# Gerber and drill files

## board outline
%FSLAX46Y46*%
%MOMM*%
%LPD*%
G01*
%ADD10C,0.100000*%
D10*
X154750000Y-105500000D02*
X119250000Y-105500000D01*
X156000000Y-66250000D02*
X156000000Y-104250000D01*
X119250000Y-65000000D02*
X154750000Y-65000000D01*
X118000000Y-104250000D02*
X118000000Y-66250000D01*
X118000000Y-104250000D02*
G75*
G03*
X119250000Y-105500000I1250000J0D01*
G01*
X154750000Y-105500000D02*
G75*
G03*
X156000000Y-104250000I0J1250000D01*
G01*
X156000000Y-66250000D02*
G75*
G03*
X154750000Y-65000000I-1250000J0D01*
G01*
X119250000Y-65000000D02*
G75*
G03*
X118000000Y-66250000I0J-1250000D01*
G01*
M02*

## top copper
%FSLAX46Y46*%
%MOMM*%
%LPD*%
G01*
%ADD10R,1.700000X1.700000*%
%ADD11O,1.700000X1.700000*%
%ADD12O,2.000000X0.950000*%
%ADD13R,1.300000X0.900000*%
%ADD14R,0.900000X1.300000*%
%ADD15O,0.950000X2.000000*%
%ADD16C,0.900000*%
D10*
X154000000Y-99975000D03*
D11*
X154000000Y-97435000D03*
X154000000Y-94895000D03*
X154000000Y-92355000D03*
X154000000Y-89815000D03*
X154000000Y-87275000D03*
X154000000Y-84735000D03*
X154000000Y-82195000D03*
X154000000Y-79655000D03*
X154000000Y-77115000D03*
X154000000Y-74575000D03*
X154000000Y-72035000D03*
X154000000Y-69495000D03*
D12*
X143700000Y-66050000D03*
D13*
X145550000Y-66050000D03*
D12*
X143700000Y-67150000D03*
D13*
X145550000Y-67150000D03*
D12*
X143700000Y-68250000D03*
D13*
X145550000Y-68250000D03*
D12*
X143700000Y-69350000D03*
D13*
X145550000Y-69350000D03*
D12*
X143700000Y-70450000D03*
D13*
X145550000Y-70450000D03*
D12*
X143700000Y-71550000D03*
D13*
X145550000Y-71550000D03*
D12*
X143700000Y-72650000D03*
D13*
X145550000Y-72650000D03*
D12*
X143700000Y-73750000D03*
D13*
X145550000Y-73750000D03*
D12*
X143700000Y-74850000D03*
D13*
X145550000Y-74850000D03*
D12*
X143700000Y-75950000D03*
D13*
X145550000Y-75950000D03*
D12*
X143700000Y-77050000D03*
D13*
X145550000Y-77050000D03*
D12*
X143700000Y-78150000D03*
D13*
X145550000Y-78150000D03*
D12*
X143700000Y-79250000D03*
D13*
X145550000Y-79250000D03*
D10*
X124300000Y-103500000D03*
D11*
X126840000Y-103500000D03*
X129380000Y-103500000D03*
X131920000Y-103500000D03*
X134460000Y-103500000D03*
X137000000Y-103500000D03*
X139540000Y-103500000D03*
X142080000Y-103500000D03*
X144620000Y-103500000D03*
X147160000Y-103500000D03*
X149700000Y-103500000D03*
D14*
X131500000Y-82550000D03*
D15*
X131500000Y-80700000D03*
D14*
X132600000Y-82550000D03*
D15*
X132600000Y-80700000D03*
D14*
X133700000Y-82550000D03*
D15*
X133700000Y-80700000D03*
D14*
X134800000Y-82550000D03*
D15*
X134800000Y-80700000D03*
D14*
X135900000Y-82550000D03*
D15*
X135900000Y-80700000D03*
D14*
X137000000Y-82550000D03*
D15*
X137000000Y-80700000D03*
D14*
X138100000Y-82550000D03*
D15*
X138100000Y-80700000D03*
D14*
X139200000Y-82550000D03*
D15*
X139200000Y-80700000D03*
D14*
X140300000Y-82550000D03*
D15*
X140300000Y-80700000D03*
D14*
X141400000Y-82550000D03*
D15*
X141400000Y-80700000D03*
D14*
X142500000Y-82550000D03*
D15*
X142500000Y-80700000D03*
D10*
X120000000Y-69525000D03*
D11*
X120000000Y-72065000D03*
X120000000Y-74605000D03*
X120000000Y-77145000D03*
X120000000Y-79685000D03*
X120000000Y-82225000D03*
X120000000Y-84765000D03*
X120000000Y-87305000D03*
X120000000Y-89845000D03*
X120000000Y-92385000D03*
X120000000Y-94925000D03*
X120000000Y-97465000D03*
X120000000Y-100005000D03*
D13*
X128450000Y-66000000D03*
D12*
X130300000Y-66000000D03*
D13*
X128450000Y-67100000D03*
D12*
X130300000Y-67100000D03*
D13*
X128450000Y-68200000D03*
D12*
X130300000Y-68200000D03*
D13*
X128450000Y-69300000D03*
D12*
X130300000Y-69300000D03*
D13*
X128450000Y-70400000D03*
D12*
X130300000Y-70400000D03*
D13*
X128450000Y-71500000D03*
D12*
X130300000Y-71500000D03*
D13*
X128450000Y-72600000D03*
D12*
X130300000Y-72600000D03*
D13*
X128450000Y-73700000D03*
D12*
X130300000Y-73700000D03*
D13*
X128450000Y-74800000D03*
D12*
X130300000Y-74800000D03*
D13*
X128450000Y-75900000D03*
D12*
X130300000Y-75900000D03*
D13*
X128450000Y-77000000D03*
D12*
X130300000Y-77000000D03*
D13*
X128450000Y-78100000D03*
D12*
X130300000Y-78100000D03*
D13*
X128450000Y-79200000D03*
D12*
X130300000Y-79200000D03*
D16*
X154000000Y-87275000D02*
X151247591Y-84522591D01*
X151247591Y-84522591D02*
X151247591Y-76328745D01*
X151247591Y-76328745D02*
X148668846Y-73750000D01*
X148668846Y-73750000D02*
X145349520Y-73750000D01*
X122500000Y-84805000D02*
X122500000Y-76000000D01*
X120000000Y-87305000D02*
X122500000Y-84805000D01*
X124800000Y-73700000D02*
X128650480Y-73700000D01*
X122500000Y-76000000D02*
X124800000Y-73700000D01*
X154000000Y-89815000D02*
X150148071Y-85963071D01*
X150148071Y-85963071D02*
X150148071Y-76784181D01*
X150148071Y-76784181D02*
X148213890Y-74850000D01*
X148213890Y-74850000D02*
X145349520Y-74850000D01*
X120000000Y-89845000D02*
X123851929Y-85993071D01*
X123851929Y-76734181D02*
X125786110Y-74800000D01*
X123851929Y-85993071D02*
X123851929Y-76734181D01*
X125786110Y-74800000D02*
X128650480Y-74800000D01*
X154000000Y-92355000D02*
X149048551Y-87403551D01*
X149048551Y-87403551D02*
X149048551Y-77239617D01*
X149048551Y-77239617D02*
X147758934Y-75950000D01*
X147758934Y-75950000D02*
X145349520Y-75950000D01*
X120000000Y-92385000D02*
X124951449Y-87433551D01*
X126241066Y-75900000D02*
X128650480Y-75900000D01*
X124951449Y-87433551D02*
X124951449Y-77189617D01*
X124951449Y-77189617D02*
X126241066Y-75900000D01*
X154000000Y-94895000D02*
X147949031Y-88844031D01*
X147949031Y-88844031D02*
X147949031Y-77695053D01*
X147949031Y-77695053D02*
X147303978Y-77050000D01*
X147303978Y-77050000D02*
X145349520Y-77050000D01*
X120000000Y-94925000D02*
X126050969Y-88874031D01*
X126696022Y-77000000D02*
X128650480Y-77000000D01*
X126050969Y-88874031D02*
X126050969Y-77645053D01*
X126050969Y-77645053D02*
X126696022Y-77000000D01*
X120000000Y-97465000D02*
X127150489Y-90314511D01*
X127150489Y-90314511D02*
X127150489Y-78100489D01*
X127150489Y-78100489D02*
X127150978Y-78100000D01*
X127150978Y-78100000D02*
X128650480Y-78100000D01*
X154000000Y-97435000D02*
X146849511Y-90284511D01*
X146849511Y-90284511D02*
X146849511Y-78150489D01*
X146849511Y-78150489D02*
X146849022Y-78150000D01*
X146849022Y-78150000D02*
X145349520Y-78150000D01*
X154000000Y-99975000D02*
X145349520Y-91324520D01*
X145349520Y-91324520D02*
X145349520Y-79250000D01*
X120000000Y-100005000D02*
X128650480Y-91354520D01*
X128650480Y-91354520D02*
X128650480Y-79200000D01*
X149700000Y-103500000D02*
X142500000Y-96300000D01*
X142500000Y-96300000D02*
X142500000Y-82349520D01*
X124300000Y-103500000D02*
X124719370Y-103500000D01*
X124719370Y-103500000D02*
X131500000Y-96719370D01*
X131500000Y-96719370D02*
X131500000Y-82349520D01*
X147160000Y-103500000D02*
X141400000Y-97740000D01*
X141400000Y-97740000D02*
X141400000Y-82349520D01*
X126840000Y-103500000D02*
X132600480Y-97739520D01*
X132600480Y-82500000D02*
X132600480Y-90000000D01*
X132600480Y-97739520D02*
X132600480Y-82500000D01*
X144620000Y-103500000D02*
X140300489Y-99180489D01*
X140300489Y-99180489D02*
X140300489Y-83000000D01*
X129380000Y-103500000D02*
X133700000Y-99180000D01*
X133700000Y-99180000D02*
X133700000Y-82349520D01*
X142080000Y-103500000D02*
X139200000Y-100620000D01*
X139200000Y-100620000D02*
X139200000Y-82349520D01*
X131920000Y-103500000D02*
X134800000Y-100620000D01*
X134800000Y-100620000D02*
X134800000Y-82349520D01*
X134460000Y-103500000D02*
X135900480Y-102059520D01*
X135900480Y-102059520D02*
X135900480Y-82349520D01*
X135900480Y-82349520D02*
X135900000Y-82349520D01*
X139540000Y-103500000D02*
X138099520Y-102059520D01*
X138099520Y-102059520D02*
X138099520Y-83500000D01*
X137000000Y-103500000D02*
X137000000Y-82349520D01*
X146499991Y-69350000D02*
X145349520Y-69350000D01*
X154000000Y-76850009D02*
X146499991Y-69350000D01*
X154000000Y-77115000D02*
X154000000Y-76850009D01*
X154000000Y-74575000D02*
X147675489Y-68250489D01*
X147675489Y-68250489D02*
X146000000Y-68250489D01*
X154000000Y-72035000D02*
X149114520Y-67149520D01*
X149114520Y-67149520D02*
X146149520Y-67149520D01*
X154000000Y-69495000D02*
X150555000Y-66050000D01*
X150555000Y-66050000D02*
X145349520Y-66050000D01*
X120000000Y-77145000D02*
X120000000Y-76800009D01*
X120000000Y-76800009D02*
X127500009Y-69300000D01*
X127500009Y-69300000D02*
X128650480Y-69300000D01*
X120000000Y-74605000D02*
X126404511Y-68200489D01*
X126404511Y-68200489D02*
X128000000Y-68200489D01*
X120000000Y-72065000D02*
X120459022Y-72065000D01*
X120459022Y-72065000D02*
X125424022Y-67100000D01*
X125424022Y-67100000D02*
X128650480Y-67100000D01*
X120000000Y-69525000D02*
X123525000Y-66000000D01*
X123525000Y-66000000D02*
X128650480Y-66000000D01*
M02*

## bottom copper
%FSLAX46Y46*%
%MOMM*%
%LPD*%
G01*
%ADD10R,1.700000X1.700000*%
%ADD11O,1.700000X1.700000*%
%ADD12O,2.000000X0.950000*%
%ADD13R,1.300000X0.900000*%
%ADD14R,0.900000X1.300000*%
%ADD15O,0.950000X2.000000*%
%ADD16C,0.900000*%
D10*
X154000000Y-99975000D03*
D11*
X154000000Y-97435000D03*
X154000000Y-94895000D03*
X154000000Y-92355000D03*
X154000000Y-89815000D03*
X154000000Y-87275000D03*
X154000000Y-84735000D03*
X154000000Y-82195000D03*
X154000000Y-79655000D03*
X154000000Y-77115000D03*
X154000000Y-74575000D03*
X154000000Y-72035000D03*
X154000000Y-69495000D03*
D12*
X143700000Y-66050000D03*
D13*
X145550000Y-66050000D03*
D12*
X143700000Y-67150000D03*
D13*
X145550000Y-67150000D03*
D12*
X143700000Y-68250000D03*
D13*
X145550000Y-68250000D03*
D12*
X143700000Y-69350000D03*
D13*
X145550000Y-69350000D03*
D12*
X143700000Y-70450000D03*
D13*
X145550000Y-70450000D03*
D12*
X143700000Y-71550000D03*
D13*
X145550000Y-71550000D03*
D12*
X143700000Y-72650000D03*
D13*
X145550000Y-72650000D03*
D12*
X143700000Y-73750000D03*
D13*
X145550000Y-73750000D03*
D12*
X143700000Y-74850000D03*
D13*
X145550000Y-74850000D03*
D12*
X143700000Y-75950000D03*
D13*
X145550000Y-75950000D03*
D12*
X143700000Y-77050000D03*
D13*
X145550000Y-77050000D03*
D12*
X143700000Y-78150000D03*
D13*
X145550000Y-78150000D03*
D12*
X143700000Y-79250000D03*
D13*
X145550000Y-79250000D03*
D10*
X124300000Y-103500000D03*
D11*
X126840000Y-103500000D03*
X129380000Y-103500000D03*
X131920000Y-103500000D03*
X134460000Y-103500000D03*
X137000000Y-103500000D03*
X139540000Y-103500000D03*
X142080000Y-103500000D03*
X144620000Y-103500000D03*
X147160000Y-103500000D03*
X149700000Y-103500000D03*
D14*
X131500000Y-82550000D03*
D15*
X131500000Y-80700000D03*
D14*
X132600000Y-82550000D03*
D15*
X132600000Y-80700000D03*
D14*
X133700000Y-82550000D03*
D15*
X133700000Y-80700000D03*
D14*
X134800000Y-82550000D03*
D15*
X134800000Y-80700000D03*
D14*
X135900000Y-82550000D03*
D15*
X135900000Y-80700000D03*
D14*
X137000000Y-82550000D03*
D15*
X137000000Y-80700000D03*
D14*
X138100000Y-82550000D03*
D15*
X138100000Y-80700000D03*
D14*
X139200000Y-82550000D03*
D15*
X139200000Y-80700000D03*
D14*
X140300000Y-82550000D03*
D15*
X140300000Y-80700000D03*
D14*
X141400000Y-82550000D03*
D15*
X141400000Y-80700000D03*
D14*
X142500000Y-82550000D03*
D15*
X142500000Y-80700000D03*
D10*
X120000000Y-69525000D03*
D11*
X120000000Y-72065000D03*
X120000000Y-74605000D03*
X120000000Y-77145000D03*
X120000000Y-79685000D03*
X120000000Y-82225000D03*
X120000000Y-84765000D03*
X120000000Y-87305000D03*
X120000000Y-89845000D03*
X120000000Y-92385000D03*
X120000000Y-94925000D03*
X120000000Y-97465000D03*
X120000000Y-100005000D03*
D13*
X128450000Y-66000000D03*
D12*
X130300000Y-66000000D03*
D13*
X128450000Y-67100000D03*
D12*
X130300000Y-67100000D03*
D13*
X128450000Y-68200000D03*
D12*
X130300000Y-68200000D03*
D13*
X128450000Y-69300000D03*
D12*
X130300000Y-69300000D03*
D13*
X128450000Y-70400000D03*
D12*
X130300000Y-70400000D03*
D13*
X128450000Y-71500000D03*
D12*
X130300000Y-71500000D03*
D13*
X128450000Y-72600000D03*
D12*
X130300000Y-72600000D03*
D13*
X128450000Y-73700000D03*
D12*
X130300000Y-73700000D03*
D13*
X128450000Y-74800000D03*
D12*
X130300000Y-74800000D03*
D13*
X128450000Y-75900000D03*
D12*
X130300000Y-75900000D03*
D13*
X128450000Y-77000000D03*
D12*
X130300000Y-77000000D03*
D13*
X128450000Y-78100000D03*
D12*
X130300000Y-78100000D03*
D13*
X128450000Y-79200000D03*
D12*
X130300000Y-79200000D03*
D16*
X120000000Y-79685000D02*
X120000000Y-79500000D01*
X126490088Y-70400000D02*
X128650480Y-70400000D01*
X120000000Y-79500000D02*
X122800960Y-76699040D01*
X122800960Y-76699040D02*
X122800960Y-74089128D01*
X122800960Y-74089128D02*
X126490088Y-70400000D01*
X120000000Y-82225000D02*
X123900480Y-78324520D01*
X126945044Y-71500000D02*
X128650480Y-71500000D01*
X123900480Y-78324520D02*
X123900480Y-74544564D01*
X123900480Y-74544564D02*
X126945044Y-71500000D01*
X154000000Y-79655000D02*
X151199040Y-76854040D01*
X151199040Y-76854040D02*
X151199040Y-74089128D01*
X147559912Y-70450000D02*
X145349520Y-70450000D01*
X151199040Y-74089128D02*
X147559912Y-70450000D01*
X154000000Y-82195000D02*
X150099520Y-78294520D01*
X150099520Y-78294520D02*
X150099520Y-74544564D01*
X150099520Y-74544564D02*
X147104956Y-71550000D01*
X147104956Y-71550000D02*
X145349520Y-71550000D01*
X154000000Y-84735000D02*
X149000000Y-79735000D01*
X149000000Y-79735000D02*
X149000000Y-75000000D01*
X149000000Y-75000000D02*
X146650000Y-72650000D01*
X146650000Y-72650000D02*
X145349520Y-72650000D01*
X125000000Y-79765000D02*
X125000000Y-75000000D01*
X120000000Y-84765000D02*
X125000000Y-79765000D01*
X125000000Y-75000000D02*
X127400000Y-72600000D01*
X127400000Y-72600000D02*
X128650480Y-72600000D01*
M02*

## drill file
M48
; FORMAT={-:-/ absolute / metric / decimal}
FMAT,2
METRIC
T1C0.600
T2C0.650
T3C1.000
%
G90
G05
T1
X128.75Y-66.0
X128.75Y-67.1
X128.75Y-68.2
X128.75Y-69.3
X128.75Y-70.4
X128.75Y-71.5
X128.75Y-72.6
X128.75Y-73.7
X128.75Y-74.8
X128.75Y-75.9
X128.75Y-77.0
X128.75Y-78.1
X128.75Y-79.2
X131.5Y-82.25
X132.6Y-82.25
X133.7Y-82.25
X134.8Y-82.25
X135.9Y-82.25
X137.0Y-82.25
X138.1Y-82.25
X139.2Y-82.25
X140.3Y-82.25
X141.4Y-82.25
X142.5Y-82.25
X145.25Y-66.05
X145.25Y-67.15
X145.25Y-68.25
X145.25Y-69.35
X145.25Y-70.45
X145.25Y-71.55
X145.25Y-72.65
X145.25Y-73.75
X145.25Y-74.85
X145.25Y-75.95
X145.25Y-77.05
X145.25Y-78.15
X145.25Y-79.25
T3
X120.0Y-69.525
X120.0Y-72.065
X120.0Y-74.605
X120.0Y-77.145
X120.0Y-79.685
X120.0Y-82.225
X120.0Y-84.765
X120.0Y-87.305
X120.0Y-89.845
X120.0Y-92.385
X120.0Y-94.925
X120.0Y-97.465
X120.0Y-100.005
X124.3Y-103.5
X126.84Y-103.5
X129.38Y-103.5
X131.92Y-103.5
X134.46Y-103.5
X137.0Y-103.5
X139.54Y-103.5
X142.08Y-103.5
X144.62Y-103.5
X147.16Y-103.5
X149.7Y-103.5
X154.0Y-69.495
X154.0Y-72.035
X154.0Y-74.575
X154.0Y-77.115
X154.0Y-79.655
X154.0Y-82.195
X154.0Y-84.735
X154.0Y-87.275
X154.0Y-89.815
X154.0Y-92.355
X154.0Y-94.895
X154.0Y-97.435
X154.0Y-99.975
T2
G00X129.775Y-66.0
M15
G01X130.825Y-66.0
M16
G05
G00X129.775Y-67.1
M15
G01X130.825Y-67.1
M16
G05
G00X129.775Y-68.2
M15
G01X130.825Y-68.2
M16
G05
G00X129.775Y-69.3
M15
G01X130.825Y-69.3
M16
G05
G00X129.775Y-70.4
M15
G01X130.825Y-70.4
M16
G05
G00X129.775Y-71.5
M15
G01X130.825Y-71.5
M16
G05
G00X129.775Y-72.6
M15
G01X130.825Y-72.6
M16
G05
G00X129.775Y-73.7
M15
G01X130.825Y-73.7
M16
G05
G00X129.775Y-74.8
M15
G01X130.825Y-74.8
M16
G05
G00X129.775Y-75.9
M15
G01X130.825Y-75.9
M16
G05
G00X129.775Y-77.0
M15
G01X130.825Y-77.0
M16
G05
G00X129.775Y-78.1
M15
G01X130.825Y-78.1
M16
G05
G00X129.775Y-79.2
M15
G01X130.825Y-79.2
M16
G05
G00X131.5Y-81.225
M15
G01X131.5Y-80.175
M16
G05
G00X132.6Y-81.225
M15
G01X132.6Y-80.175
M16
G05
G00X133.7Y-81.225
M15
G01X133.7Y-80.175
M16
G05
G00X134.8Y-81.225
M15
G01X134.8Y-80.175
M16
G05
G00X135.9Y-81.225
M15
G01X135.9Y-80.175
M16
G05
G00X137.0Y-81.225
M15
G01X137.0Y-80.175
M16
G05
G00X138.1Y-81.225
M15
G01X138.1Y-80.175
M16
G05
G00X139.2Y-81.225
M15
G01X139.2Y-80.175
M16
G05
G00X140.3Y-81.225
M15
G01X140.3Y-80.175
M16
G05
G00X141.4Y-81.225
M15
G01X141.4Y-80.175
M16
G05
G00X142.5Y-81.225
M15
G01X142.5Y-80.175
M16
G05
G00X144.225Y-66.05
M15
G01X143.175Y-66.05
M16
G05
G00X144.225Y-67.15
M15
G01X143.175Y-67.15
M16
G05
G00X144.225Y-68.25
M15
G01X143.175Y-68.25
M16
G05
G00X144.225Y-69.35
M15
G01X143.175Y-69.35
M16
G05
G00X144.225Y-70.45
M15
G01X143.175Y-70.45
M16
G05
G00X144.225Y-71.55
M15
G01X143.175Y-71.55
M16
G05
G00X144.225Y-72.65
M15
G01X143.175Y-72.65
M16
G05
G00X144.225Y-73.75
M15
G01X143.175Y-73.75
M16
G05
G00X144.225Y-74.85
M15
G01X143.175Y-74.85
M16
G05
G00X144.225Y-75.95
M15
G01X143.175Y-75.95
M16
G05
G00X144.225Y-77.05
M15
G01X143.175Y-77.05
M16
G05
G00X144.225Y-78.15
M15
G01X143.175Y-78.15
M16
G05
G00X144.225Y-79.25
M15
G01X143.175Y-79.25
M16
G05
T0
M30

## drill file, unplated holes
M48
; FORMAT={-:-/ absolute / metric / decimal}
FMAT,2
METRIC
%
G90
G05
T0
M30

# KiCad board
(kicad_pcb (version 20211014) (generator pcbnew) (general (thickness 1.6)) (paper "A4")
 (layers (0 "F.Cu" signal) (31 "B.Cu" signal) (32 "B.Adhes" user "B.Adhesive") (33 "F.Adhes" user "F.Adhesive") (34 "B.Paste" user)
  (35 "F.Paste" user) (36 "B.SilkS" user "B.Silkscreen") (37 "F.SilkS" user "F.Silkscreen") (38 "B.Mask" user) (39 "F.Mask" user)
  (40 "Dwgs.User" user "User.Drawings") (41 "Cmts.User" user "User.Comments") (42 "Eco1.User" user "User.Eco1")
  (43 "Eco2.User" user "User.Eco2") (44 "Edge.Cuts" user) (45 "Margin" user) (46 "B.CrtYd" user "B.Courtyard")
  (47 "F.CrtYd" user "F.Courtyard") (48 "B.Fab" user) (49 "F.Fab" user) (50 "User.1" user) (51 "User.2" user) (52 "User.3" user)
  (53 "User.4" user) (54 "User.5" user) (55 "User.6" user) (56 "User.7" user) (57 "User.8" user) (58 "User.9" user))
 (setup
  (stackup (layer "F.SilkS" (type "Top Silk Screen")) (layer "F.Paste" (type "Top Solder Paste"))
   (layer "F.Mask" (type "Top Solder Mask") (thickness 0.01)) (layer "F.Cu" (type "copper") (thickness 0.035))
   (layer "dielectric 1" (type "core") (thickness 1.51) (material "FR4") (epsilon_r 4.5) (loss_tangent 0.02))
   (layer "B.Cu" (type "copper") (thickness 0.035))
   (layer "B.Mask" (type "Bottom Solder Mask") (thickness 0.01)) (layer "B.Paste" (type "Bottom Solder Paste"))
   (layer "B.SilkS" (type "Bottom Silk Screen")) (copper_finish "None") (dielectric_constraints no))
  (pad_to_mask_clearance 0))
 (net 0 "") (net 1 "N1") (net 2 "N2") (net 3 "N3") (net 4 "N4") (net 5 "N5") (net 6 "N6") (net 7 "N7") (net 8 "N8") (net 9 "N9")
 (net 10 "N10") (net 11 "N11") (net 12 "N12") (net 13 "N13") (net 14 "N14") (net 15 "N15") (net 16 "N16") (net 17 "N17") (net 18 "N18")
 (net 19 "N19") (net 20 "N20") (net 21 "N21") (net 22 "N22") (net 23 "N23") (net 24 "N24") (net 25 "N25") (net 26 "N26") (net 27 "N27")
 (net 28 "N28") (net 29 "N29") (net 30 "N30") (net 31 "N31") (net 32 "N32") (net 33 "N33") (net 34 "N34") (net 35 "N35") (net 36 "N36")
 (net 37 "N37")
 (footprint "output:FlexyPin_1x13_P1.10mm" (layer "F.Cu") (at 128.75 66)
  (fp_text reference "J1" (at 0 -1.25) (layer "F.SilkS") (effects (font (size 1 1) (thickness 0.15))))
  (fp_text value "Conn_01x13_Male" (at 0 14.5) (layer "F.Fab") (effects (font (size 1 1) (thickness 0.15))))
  (pad "" thru_hole oval locked (at 1.55 12.1) (size 2 0.95) (drill oval 1.7 0.65) (layers *.Cu *.Mask))
  (pad "" thru_hole oval locked (at 1.55 5.5) (size 2 0.95) (drill oval 1.7 0.65) (layers *.Cu *.Mask))
  (pad "" thru_hole oval locked (at 1.55 13.2) (size 2 0.95) (drill oval 1.7 0.65) (layers *.Cu *.Mask))
  (pad "" thru_hole oval locked (at 1.55 8.8) (size 2 0.95) (drill oval 1.7 0.65) (layers *.Cu *.Mask))
  (pad "" thru_hole oval locked (at 1.55 4.4) (size 2 0.95) (drill oval 1.7 0.65) (layers *.Cu *.Mask))
  (pad "" thru_hole oval locked (at 1.55 9.9) (size 2 0.95) (drill oval 1.7 0.65) (layers *.Cu *.Mask))
  (pad "" thru_hole oval locked (at 1.55 3.3) (size 2 0.95) (drill oval 1.7 0.65) (layers *.Cu *.Mask))
  (pad "" thru_hole oval locked (at 1.55 0) (size 2 0.95) (drill oval 1.7 0.65) (layers *.Cu *.Mask))
  (pad "" thru_hole oval locked (at 1.55 2.2) (size 2 0.95) (drill oval 1.7 0.65) (layers *.Cu *.Mask))
  (pad "" thru_hole oval locked (at 1.55 1.1) (size 2 0.95) (drill oval 1.7 0.65) (layers *.Cu *.Mask))
  (pad "" thru_hole oval locked (at 1.55 11) (size 2 0.95) (drill oval 1.7 0.65) (layers *.Cu *.Mask))
  (pad "" thru_hole oval locked (at 1.55 6.6) (size 2 0.95) (drill oval 1.7 0.65) (layers *.Cu *.Mask))
  (pad "" thru_hole oval locked (at 1.55 7.7) (size 2 0.95) (drill oval 1.7 0.65) (layers *.Cu *.Mask))
  (pad "1" thru_hole rect locked (at 0 0) (size 1.3 0.9) (drill 0.6 (offset -0.3 0)) (layers *.Cu *.Mask) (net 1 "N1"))
  (pad "2" thru_hole rect locked (at 0 1.1) (size 1.3 0.9) (drill 0.6 (offset -0.3 0)) (layers *.Cu *.Mask) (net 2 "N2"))
  (pad "3" thru_hole rect locked (at 0 2.2) (size 1.3 0.9) (drill 0.6 (offset -0.3 0)) (layers *.Cu *.Mask) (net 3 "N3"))
  (pad "4" thru_hole rect locked (at 0 3.3) (size 1.3 0.9) (drill 0.6 (offset -0.3 0)) (layers *.Cu *.Mask) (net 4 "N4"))
  (pad "5" thru_hole rect locked (at 0 4.4) (size 1.3 0.9) (drill 0.6 (offset -0.3 0)) (layers *.Cu *.Mask) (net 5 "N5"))
  (pad "6" thru_hole rect locked (at 0 5.5) (size 1.3 0.9) (drill 0.6 (offset -0.3 0)) (layers *.Cu *.Mask) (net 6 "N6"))
  (pad "7" thru_hole rect locked (at 0 6.6) (size 1.3 0.9) (drill 0.6 (offset -0.3 0)) (layers *.Cu *.Mask) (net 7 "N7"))
  (pad "8" thru_hole rect locked (at 0 7.7) (size 1.3 0.9) (drill 0.6 (offset -0.3 0)) (layers *.Cu *.Mask) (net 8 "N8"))
  (pad "9" thru_hole rect locked (at 0 8.8) (size 1.3 0.9) (drill 0.6 (offset -0.3 0)) (layers *.Cu *.Mask) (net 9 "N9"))
  (pad "10" thru_hole rect locked (at 0 9.9) (size 1.3 0.9) (drill 0.6 (offset -0.3 0)) (layers *.Cu *.Mask) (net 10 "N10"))
  (pad "11" thru_hole rect locked (at 0 11) (size 1.3 0.9) (drill 0.6 (offset -0.3 0)) (layers *.Cu *.Mask) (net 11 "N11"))
  (pad "12" thru_hole rect locked (at 0 12.1) (size 1.3 0.9) (drill 0.6 (offset -0.3 0)) (layers *.Cu *.Mask) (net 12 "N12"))
  (pad "13" thru_hole rect locked (at 0 13.2) (size 1.3 0.9) (drill 0.6 (offset -0.3 0)) (layers *.Cu *.Mask) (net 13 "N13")))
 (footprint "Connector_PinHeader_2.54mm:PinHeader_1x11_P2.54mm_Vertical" (layer "F.Cu") (at 124.3 103.5 90)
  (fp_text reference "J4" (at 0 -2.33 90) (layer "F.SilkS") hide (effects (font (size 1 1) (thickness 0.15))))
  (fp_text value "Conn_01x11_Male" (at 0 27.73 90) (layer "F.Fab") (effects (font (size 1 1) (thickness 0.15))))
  (pad "1" thru_hole rect (at 0 0 90) (size 1.7 1.7) (drill 1) (layers *.Cu *.Mask) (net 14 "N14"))
  (pad "2" thru_hole oval (at 0 2.54 90) (size 1.7 1.7) (drill 1) (layers *.Cu *.Mask) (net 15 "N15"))
  (pad "3" thru_hole oval (at 0 5.08 90) (size 1.7 1.7) (drill 1) (layers *.Cu *.Mask) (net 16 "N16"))
  (pad "4" thru_hole oval (at 0 7.62 90) (size 1.7 1.7) (drill 1) (layers *.Cu *.Mask) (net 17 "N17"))
  (pad "5" thru_hole oval (at 0 10.16 90) (size 1.7 1.7) (drill 1) (layers *.Cu *.Mask) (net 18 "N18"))
  (pad "6" thru_hole oval (at 0 12.7 90) (size 1.7 1.7) (drill 1) (layers *.Cu *.Mask) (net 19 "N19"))
  (pad "7" thru_hole oval (at 0 15.24 90) (size 1.7 1.7) (drill 1) (layers *.Cu *.Mask) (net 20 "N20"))
  (pad "8" thru_hole oval (at 0 17.78 90) (size 1.7 1.7) (drill 1) (layers *.Cu *.Mask) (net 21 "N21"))
  (pad "9" thru_hole oval (at 0 20.32 90) (size 1.7 1.7) (drill 1) (layers *.Cu *.Mask) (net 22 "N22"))
  (pad "10" thru_hole oval (at 0 22.86 90) (size 1.7 1.7) (drill 1) (layers *.Cu *.Mask) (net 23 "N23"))
  (pad "11" thru_hole oval (at 0 25.4 90) (size 1.7 1.7) (drill 1) (layers *.Cu *.Mask) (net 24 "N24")))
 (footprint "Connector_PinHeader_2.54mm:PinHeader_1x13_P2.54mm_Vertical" (layer "F.Cu") (at 120 69.525)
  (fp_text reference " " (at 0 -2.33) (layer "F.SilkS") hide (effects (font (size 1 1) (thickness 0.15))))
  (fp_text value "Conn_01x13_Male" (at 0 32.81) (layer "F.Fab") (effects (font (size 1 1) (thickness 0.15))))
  (pad "1" thru_hole rect (at 0 0) (size 1.7 1.7) (drill 1) (layers *.Cu *.Mask) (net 1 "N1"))
  (pad "2" thru_hole oval (at 0 2.54) (size 1.7 1.7) (drill 1) (layers *.Cu *.Mask) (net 2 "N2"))
  (pad "3" thru_hole oval (at 0 5.08) (size 1.7 1.7) (drill 1) (layers *.Cu *.Mask) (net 3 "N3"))
  (pad "4" thru_hole oval (at 0 7.62) (size 1.7 1.7) (drill 1) (layers *.Cu *.Mask) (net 4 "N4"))
  (pad "5" thru_hole oval (at 0 10.16) (size 1.7 1.7) (drill 1) (layers *.Cu *.Mask) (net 5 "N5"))
  (pad "6" thru_hole oval (at 0 12.7) (size 1.7 1.7) (drill 1) (layers *.Cu *.Mask) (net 6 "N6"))
  (pad "7" thru_hole oval (at 0 15.24) (size 1.7 1.7) (drill 1) (layers *.Cu *.Mask) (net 7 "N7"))
  (pad "8" thru_hole oval (at 0 17.78) (size 1.7 1.7) (drill 1) (layers *.Cu *.Mask) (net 8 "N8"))
  (pad "9" thru_hole oval (at 0 20.32) (size 1.7 1.7) (drill 1) (layers *.Cu *.Mask) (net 9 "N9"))
  (pad "10" thru_hole oval (at 0 22.86) (size 1.7 1.7) (drill 1) (layers *.Cu *.Mask) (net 10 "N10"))
  (pad "11" thru_hole oval (at 0 25.4) (size 1.7 1.7) (drill 1) (layers *.Cu *.Mask) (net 11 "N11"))
  (pad "12" thru_hole oval (at 0 27.94) (size 1.7 1.7) (drill 1) (layers *.Cu *.Mask) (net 12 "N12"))
  (pad "13" thru_hole oval (at 0 30.48) (size 1.7 1.7) (drill 1) (layers *.Cu *.Mask) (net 13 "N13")))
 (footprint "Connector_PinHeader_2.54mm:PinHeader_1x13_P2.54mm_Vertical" (layer "F.Cu") (at 154 99.975 180)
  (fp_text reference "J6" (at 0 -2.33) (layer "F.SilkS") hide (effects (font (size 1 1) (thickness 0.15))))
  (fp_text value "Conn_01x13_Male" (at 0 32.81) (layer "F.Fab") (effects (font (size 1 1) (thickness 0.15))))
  (pad "1" thru_hole rect (at 0 0 180) (size 1.7 1.7) (drill 1) (layers *.Cu *.Mask) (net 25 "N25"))
  (pad "2" thru_hole oval (at 0 2.54 180) (size 1.7 1.7) (drill 1) (layers *.Cu *.Mask) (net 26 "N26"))
  (pad "3" thru_hole oval (at 0 5.08 180) (size 1.7 1.7) (drill 1) (layers *.Cu *.Mask) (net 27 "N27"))
  (pad "4" thru_hole oval (at 0 7.62 180) (size 1.7 1.7) (drill 1) (layers *.Cu *.Mask) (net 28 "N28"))
  (pad "5" thru_hole oval (at 0 10.16 180) (size 1.7 1.7) (drill 1) (layers *.Cu *.Mask) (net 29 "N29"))
  (pad "6" thru_hole oval (at 0 12.7 180) (size 1.7 1.7) (drill 1) (layers *.Cu *.Mask) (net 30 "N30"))
  (pad "7" thru_hole oval (at 0 15.24 180) (size 1.7 1.7) (drill 1) (layers *.Cu *.Mask) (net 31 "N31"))
  (pad "8" thru_hole oval (at 0 17.78 180) (size 1.7 1.7) (drill 1) (layers *.Cu *.Mask) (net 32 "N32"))
  (pad "9" thru_hole oval (at 0 20.32 180) (size 1.7 1.7) (drill 1) (layers *.Cu *.Mask) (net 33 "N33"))
  (pad "10" thru_hole oval (at 0 22.86 180) (size 1.7 1.7) (drill 1) (layers *.Cu *.Mask) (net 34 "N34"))
  (pad "11" thru_hole oval (at 0 25.4 180) (size 1.7 1.7) (drill 1) (layers *.Cu *.Mask) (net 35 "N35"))
  (pad "12" thru_hole oval (at 0 27.94 180) (size 1.7 1.7) (drill 1) (layers *.Cu *.Mask) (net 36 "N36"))
  (pad "13" thru_hole oval (at 0 30.48 180) (size 1.7 1.7) (drill 1) (layers *.Cu *.Mask) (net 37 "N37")))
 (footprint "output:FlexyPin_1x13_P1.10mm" (layer "F.Cu") (at 145.25 79.25 180)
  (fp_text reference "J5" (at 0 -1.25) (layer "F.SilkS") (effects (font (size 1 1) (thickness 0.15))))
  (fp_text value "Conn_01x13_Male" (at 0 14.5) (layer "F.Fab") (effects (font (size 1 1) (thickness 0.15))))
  (pad "" thru_hole oval locked (at 1.55 11 180) (size 2 0.95) (drill oval 1.7 0.65) (layers *.Cu *.Mask))
  (pad "" thru_hole oval locked (at 1.55 8.8 180) (size 2 0.95) (drill oval 1.7 0.65) (layers *.Cu *.Mask))
  (pad "" thru_hole oval locked (at 1.55 5.5 180) (size 2 0.95) (drill oval 1.7 0.65) (layers *.Cu *.Mask))
  (pad "" thru_hole oval locked (at 1.55 13.2 180) (size 2 0.95) (drill oval 1.7 0.65) (layers *.Cu *.Mask))
  (pad "" thru_hole oval locked (at 1.55 4.4 180) (size 2 0.95) (drill oval 1.7 0.65) (layers *.Cu *.Mask))
  (pad "" thru_hole oval locked (at 1.55 3.3 180) (size 2 0.95) (drill oval 1.7 0.65) (layers *.Cu *.Mask))
  (pad "" thru_hole oval locked (at 1.55 0 180) (size 2 0.95) (drill oval 1.7 0.65) (layers *.Cu *.Mask))
  (pad "" thru_hole oval locked (at 1.55 9.9 180) (size 2 0.95) (drill oval 1.7 0.65) (layers *.Cu *.Mask))
  (pad "" thru_hole oval locked (at 1.55 12.1 180) (size 2 0.95) (drill oval 1.7 0.65) (layers *.Cu *.Mask))
  (pad "" thru_hole oval locked (at 1.55 7.7 180) (size 2 0.95) (drill oval 1.7 0.65) (layers *.Cu *.Mask))
  (pad "" thru_hole oval locked (at 1.55 2.2 180) (size 2 0.95) (drill oval 1.7 0.65) (layers *.Cu *.Mask))
  (pad "" thru_hole oval locked (at 1.55 6.6 180) (size 2 0.95) (drill oval 1.7 0.65) (layers *.Cu *.Mask))
  (pad "" thru_hole oval locked (at 1.55 1.1 180) (size 2 0.95) (drill oval 1.7 0.65) (layers *.Cu *.Mask))
  (pad "1" thru_hole rect locked (at 0 0 180) (size 1.3 0.9) (drill 0.6 (offset -0.3 0)) (layers *.Cu *.Mask) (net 25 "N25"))
  (pad "2" thru_hole rect locked (at 0 1.1 180) (size 1.3 0.9) (drill 0.6 (offset -0.3 0)) (layers *.Cu *.Mask) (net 26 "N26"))
  (pad "3" thru_hole rect locked (at 0 2.2 180) (size 1.3 0.9) (drill 0.6 (offset -0.3 0)) (layers *.Cu *.Mask) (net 27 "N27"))
  (pad "4" thru_hole rect locked (at 0 3.3 180) (size 1.3 0.9) (drill 0.6 (offset -0.3 0)) (layers *.Cu *.Mask) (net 28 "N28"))
  (pad "5" thru_hole rect locked (at 0 4.4 180) (size 1.3 0.9) (drill 0.6 (offset -0.3 0)) (layers *.Cu *.Mask) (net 29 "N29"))
  (pad "6" thru_hole rect locked (at 0 5.5 180) (size 1.3 0.9) (drill 0.6 (offset -0.3 0)) (layers *.Cu *.Mask) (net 30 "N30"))
  (pad "7" thru_hole rect locked (at 0 6.6 180) (size 1.3 0.9) (drill 0.6 (offset -0.3 0)) (layers *.Cu *.Mask) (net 31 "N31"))
  (pad "8" thru_hole rect locked (at 0 7.7 180) (size 1.3 0.9) (drill 0.6 (offset -0.3 0)) (layers *.Cu *.Mask) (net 32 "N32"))
  (pad "9" thru_hole rect locked (at 0 8.8 180) (size 1.3 0.9) (drill 0.6 (offset -0.3 0)) (layers *.Cu *.Mask) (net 33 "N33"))
  (pad "10" thru_hole rect locked (at 0 9.9 180) (size 1.3 0.9) (drill 0.6 (offset -0.3 0)) (layers *.Cu *.Mask) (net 34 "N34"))
  (pad "11" thru_hole rect locked (at 0 11 180) (size 1.3 0.9) (drill 0.6 (offset -0.3 0)) (layers *.Cu *.Mask) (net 35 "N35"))
  (pad "12" thru_hole rect locked (at 0 12.1 180) (size 1.3 0.9) (drill 0.6 (offset -0.3 0)) (layers *.Cu *.Mask) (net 36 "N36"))
  (pad "13" thru_hole rect locked (at 0 13.2 180) (size 1.3 0.9) (drill 0.6 (offset -0.3 0)) (layers *.Cu *.Mask) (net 37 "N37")))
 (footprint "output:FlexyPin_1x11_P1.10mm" (layer "F.Cu") (at 131.5 82.25 90)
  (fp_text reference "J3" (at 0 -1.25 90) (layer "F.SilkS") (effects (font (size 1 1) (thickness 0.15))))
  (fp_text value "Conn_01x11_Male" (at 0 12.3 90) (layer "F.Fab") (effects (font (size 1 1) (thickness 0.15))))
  (pad "" thru_hole oval locked (at 1.55 2.2 90) (size 2 0.95) (drill oval 1.7 0.65) (layers *.Cu *.Mask))
  (pad "" thru_hole oval locked (at 1.55 11 90) (size 2 0.95) (drill oval 1.7 0.65) (layers *.Cu *.Mask))
  (pad "" thru_hole oval locked (at 1.55 8.8 90) (size 2 0.95) (drill oval 1.7 0.65) (layers *.Cu *.Mask))
  (pad "" thru_hole oval locked (at 1.55 7.7 90) (size 2 0.95) (drill oval 1.7 0.65) (layers *.Cu *.Mask))
  (pad "" thru_hole oval locked (at 1.55 5.5 90) (size 2 0.95) (drill oval 1.7 0.65) (layers *.Cu *.Mask))
  (pad "" thru_hole oval locked (at 1.55 6.6 90) (size 2 0.95) (drill oval 1.7 0.65) (layers *.Cu *.Mask))
  (pad "" thru_hole oval locked (at 1.55 0 90) (size 2 0.95) (drill oval 1.7 0.65) (layers *.Cu *.Mask))
  (pad "" thru_hole oval locked (at 1.55 1.1 90) (size 2 0.95) (drill oval 1.7 0.65) (layers *.Cu *.Mask))
  (pad "" thru_hole oval locked (at 1.55 4.4 90) (size 2 0.95) (drill oval 1.7 0.65) (layers *.Cu *.Mask))
  (pad "" thru_hole oval locked (at 1.55 3.3 90) (size 2 0.95) (drill oval 1.7 0.65) (layers *.Cu *.Mask))
  (pad "" thru_hole oval locked (at 1.55 9.9 90) (size 2 0.95) (drill oval 1.7 0.65) (layers *.Cu *.Mask))
  (pad "1" thru_hole rect locked (at 0 0 90) (size 1.3 0.9) (drill 0.6 (offset -0.3 0)) (layers *.Cu *.Mask) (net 14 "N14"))
  (pad "2" thru_hole rect locked (at 0 1.1 90) (size 1.3 0.9) (drill 0.6 (offset -0.3 0)) (layers *.Cu *.Mask) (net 15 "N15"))
  (pad "3" thru_hole rect locked (at 0 2.2 90) (size 1.3 0.9) (drill 0.6 (offset -0.3 0)) (layers *.Cu *.Mask) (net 16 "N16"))
  (pad "4" thru_hole rect locked (at 0 3.3 90) (size 1.3 0.9) (drill 0.6 (offset -0.3 0)) (layers *.Cu *.Mask) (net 17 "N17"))
  (pad "5" thru_hole rect locked (at 0 4.4 90) (size 1.3 0.9) (drill 0.6 (offset -0.3 0)) (layers *.Cu *.Mask) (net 18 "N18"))
  (pad "6" thru_hole rect locked (at 0 5.5 90) (size 1.3 0.9) (drill 0.6 (offset -0.3 0)) (layers *.Cu *.Mask) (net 19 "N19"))
  (pad "7" thru_hole rect locked (at 0 6.6 90) (size 1.3 0.9) (drill 0.6 (offset -0.3 0)) (layers *.Cu *.Mask) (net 20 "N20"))
  (pad "8" thru_hole rect locked (at 0 7.7 90) (size 1.3 0.9) (drill 0.6 (offset -0.3 0)) (layers *.Cu *.Mask) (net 21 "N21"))
  (pad "9" thru_hole rect locked (at 0 8.8 90) (size 1.3 0.9) (drill 0.6 (offset -0.3 0)) (layers *.Cu *.Mask) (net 22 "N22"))
  (pad "10" thru_hole rect locked (at 0 9.9 90) (size 1.3 0.9) (drill 0.6 (offset -0.3 0)) (layers *.Cu *.Mask) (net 23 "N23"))
  (pad "11" thru_hole rect locked (at 0 11 90) (size 1.3 0.9) (drill 0.6 (offset -0.3 0)) (layers *.Cu *.Mask) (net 24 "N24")))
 (gr_arc (start 154.75 65) (mid 155.633883 65.366117) (end 156 66.25) (layer "Edge.Cuts") (width 0.1))
 (gr_line (start 156 66.25) (end 156 104.25) (layer "Edge.Cuts") (width 0.1))
 (gr_arc (start 119.25 105.5) (mid 118.366117 105.133883) (end 118 104.25) (layer "Edge.Cuts") (width 0.1))
 (gr_arc (start 156 104.25) (mid 155.633883 105.133883) (end 154.75 105.5) (layer "Edge.Cuts") (width 0.1))
 (gr_line (start 119.25 65) (end 154.75 65) (layer "Edge.Cuts") (width 0.1))
 (gr_line (start 118 104.25) (end 118 66.25) (layer "Edge.Cuts") (width 0.1))
 (gr_line (start 154.75 105.5) (end 119.25 105.5) (layer "Edge.Cuts") (width 0.1))
 (gr_arc (start 118 66.25) (mid 118.366117 65.366117) (end 119.25 65) (layer "Edge.Cuts") (width 0.1))
 (segment (start 120 69.525) (end 123.525 66) (width 0.9) (layer "F.Cu") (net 1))
 (segment (start 123.525 66) (end 128.65048 66) (width 0.9) (layer "F.Cu") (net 1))
 (segment (start 125.424022 67.1) (end 128.65048 67.1) (width 0.9) (layer "F.Cu") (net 2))
 (segment (start 120.459022 72.065) (end 125.424022 67.1) (width 0.9) (layer "F.Cu") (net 2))
 (segment (start 120 72.065) (end 120.459022 72.065) (width 0.9) (layer "F.Cu") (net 2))
 (segment (start 120 74.605) (end 126.404511 68.200489) (width 0.9) (layer "F.Cu") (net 3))
 (segment (start 126.404511 68.200489) (end 128 68.200489) (width 0.9) (layer "F.Cu") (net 3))
 (segment (start 120 76.800009) (end 127.500009 69.3) (width 0.9) (layer "F.Cu") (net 4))
 (segment (start 127.500009 69.3) (end 128.65048 69.3) (width 0.9) (layer "F.Cu") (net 4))
 (segment (start 120 77.145) (end 120 76.800009) (width 0.9) (layer "F.Cu") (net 4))
 (segment (start 122.80096 76.69904) (end 122.80096 74.089128) (width 0.9) (layer "B.Cu") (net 5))
 (segment (start 120 79.5) (end 122.80096 76.69904) (width 0.9) (layer "B.Cu") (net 5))
 (segment (start 126.490088 70.4) (end 128.65048 70.4) (width 0.9) (layer "B.Cu") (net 5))
 (segment (start 120 79.685) (end 120 79.5) (width 0.9) (layer "B.Cu") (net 5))
 (segment (start 122.80096 74.089128) (end 126.490088 70.4) (width 0.9) (layer "B.Cu") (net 5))
 (segment (start 120 82.225) (end 123.90048 78.32452) (width 0.9) (layer "B.Cu") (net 6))
 (segment (start 126.945044 71.5) (end 128.65048 71.5) (width 0.9) (layer "B.Cu") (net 6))
 (segment (start 123.90048 74.544564) (end 126.945044 71.5) (width 0.9) (layer "B.Cu") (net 6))
 (segment (start 123.90048 78.32452) (end 123.90048 74.544564) (width 0.9) (layer "B.Cu") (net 6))
 (segment (start 125 75) (end 127.4 72.6) (width 0.9) (layer "B.Cu") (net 7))
 (segment (start 125 79.765) (end 125 75) (width 0.9) (layer "B.Cu") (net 7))
 (segment (start 127.4 72.6) (end 128.65048 72.6) (width 0.9) (layer "B.Cu") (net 7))
 (segment (start 120 84.765) (end 125 79.765) (width 0.9) (layer "B.Cu") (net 7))
 (segment (start 124.8 73.7) (end 128.65048 73.7) (width 0.9) (layer "F.Cu") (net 8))
 (segment (start 120 87.305) (end 122.5 84.805) (width 0.9) (layer "F.Cu") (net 8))
 (segment (start 122.5 84.805) (end 122.5 76) (width 0.9) (layer "F.Cu") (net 8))
 (segment (start 122.5 76) (end 124.8 73.7) (width 0.9) (layer "F.Cu") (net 8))
 (segment (start 123.851929 76.734181) (end 125.78611 74.8) (width 0.9) (layer "F.Cu") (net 9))
 (segment (start 125.78611 74.8) (end 128.65048 74.8) (width 0.9) (layer "F.Cu") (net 9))
 (segment (start 123.851929 85.993071) (end 123.851929 76.734181) (width 0.9) (layer "F.Cu") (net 9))
 (segment (start 120 89.845) (end 123.851929 85.993071) (width 0.9) (layer "F.Cu") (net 9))
 (segment (start 124.951449 77.189617) (end 126.241066 75.9) (width 0.9) (layer "F.Cu") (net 10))
 (segment (start 124.951449 87.433551) (end 124.951449 77.189617) (width 0.9) (layer "F.Cu") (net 10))
 (segment (start 126.241066 75.9) (end 128.65048 75.9) (width 0.9) (layer "F.Cu") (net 10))
 (segment (start 120 92.385) (end 124.951449 87.433551) (width 0.9) (layer "F.Cu") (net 10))
 (segment (start 126.050969 88.874031) (end 126.050969 77.645053) (width 0.9) (layer "F.Cu") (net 11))
 (segment (start 120 94.925) (end 126.050969 88.874031) (width 0.9) (layer "F.Cu") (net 11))
 (segment (start 126.050969 77.645053) (end 126.696022 77) (width 0.9) (layer "F.Cu") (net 11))
 (segment (start 126.696022 77) (end 128.65048 77) (width 0.9) (layer "F.Cu") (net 11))
 (segment (start 127.150489 78.100489) (end 127.150978 78.1) (width 0.9) (layer "F.Cu") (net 12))
 (segment (start 120 97.465) (end 127.150489 90.314511) (width 0.9) (layer "F.Cu") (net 12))
 (segment (start 127.150489 90.314511) (end 127.150489 78.100489) (width 0.9) (layer "F.Cu") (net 12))
 (segment (start 127.150978 78.1) (end 128.65048 78.1) (width 0.9) (layer "F.Cu") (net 12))
 (segment (start 120 100.005) (end 128.65048 91.35452) (width 0.9) (layer "F.Cu") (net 13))
 (segment (start 128.65048 91.35452) (end 128.65048 79.2) (width 0.9) (layer "F.Cu") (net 13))
 (segment (start 124.71937 103.5) (end 131.5 96.71937) (width 0.9) (layer "F.Cu") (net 14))
 (segment (start 131.5 96.71937) (end 131.5 82.34952) (width 0.9) (layer "F.Cu") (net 14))
 (segment (start 124.3 103.5) (end 124.71937 103.5) (width 0.9) (layer "F.Cu") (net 14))
 (segment (start 132.60048 82.5) (end 132.60048 90) (width 0.9) (layer "F.Cu") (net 15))
 (segment (start 132.60048 97.73952) (end 132.60048 82.5) (width 0.9) (layer "F.Cu") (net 15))
 (segment (start 126.84 103.5) (end 132.60048 97.73952) (width 0.9) (layer "F.Cu") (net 15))
 (segment (start 129.38 103.5) (end 133.7 99.18) (width 0.9) (layer "F.Cu") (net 16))
 (segment (start 133.7 99.18) (end 133.7 82.34952) (width 0.9) (layer "F.Cu") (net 16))
 (segment (start 131.92 103.5) (end 134.8 100.62) (width 0.9) (layer "F.Cu") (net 17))
 (segment (start 134.8 100.62) (end 134.8 82.34952) (width 0.9) (layer "F.Cu") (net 17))
 (segment (start 135.90048 82.34952) (end 135.9 82.34952) (width 0.9) (layer "F.Cu") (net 18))
 (segment (start 135.90048 102.05952) (end 135.90048 82.34952) (width 0.9) (layer "F.Cu") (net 18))
 (segment (start 134.46 103.5) (end 135.90048 102.05952) (width 0.9) (layer "F.Cu") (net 18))
 (segment (start 137 103.5) (end 137 82.34952) (width 0.9) (layer "F.Cu") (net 19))
 (segment (start 138.09952 102.05952) (end 138.09952 83.5) (width 0.9) (layer "F.Cu") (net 20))
 (segment (start 139.54 103.5) (end 138.09952 102.05952) (width 0.9) (layer "F.Cu") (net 20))
 (segment (start 139.2 100.62) (end 139.2 82.34952) (width 0.9) (layer "F.Cu") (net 21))
 (segment (start 142.08 103.5) (end 139.2 100.62) (width 0.9) (layer "F.Cu") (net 21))
 (segment (start 140.300489 99.180489) (end 140.300489 83) (width 0.9) (layer "F.Cu") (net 22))
 (segment (start 144.62 103.5) (end 140.300489 99.180489) (width 0.9) (layer "F.Cu") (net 22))
 (segment (start 147.16 103.5) (end 141.4 97.74) (width 0.9) (layer "F.Cu") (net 23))
 (segment (start 141.4 97.74) (end 141.4 82.34952) (width 0.9) (layer "F.Cu") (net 23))
 (segment (start 142.5 96.3) (end 142.5 82.34952) (width 0.9) (layer "F.Cu") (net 24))
 (segment (start 149.7 103.5) (end 142.5 96.3) (width 0.9) (layer "F.Cu") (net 24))
 (segment (start 154 69.495) (end 150.555 66.05) (width 0.9) (layer "F.Cu") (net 37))
 (segment (start 150.555 66.05) (end 145.34952 66.05) (width 0.9) (layer "F.Cu") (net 37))
 (segment (start 149.11452 67.14952) (end 146.14952 67.14952) (width 0.9) (layer "F.Cu") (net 36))
 (segment (start 154 72.035) (end 149.11452 67.14952) (width 0.9) (layer "F.Cu") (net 36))
 (segment (start 147.675489 68.250489) (end 146 68.250489) (width 0.9) (layer "F.Cu") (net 35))
 (segment (start 154 74.575) (end 147.675489 68.250489) (width 0.9) (layer "F.Cu") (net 35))
 (segment (start 154 76.850009) (end 146.499991 69.35) (width 0.9) (layer "F.Cu") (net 34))
 (segment (start 154 77.115) (end 154 76.850009) (width 0.9) (layer "F.Cu") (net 34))
 (segment (start 146.499991 69.35) (end 145.34952 69.35) (width 0.9) (layer "F.Cu") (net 34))
 (segment (start 147.559912 70.45) (end 145.34952 70.45) (width 0.9) (layer "B.Cu") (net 33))
 (segment (start 151.19904 76.85404) (end 151.19904 74.089128) (width 0.9) (layer "B.Cu") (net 33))
 (segment (start 151.19904 74.089128) (end 147.559912 70.45) (width 0.9) (layer "B.Cu") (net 33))
 (segment (start 154 79.655) (end 151.19904 76.85404) (width 0.9) (layer "B.Cu") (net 33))
 (segment (start 154 82.195) (end 150.09952 78.29452) (width 0.9) (layer "B.Cu") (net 32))
 (segment (start 150.09952 78.29452) (end 150.09952 74.544564) (width 0.9) (layer "B.Cu") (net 32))
 (segment (start 147.104956 71.55) (end 145.34952 71.55) (width 0.9) (layer "B.Cu") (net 32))
 (segment (start 150.09952 74.544564) (end 147.104956 71.55) (width 0.9) (layer "B.Cu") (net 32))
 (segment (start 146.65 72.65) (end 145.34952 72.65) (width 0.9) (layer "B.Cu") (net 31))
 (segment (start 154 84.735) (end 149 79.735) (width 0.9) (layer "B.Cu") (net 31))
 (segment (start 149 79.735) (end 149 75) (width 0.9) (layer "B.Cu") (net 31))
 (segment (start 149 75) (end 146.65 72.65) (width 0.9) (layer "B.Cu") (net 31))
 (segment (start 154 87.275) (end 151.247591 84.522591) (width 0.9) (layer "F.Cu") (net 30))
 (segment (start 151.247591 76.328745) (end 148.668846 73.75) (width 0.9) (layer "F.Cu") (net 30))
 (segment (start 151.247591 84.522591) (end 151.247591 76.328745) (width 0.9) (layer "F.Cu") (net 30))
 (segment (start 148.668846 73.75) (end 145.34952 73.75) (width 0.9) (layer "F.Cu") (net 30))
 (segment (start 154 89.815) (end 150.148071 85.963071) (width 0.9) (layer "F.Cu") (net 29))
 (segment (start 150.148071 85.963071) (end 150.148071 76.784181) (width 0.9) (layer "F.Cu") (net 29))
 (segment (start 150.148071 76.784181) (end 148.21389 74.85) (width 0.9) (layer "F.Cu") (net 29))
 (segment (start 148.21389 74.85) (end 145.34952 74.85) (width 0.9) (layer "F.Cu") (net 29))
 (segment (start 154 92.355) (end 149.048551 87.403551) (width 0.9) (layer "F.Cu") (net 28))
 (segment (start 149.048551 87.403551) (end 149.048551 77.239617) (width 0.9) (layer "F.Cu") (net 28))
 (segment (start 147.758934 75.95) (end 145.34952 75.95) (width 0.9) (layer "F.Cu") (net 28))
 (segment (start 149.048551 77.239617) (end 147.758934 75.95) (width 0.9) (layer "F.Cu") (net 28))
 (segment (start 154 94.895) (end 147.949031 88.844031) (width 0.9) (layer "F.Cu") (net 27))
 (segment (start 147.949031 88.844031) (end 147.949031 77.695053) (width 0.9) (layer "F.Cu") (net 27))
 (segment (start 147.303978 77.05) (end 145.34952 77.05) (width 0.9) (layer "F.Cu") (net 27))
 (segment (start 147.949031 77.695053) (end 147.303978 77.05) (width 0.9) (layer "F.Cu") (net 27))
 (segment (start 154 97.435) (end 146.849511 90.284511) (width 0.9) (layer "F.Cu") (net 26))
 (segment (start 146.849511 90.284511) (end 146.849511 78.150489) (width 0.9) (layer "F.Cu") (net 26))
 (segment (start 146.849511 78.150489) (end 146.849022 78.15) (width 0.9) (layer "F.Cu") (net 26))
 (segment (start 146.849022 78.15) (end 145.34952 78.15) (width 0.9) (layer "F.Cu") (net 26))
 (segment (start 154 99.975) (end 145.34952 91.32452) (width 0.9) (layer "F.Cu") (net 25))
 (segment (start 145.34952 91.32452) (end 145.34952 79.25) (width 0.9) (layer "F.Cu") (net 25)))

